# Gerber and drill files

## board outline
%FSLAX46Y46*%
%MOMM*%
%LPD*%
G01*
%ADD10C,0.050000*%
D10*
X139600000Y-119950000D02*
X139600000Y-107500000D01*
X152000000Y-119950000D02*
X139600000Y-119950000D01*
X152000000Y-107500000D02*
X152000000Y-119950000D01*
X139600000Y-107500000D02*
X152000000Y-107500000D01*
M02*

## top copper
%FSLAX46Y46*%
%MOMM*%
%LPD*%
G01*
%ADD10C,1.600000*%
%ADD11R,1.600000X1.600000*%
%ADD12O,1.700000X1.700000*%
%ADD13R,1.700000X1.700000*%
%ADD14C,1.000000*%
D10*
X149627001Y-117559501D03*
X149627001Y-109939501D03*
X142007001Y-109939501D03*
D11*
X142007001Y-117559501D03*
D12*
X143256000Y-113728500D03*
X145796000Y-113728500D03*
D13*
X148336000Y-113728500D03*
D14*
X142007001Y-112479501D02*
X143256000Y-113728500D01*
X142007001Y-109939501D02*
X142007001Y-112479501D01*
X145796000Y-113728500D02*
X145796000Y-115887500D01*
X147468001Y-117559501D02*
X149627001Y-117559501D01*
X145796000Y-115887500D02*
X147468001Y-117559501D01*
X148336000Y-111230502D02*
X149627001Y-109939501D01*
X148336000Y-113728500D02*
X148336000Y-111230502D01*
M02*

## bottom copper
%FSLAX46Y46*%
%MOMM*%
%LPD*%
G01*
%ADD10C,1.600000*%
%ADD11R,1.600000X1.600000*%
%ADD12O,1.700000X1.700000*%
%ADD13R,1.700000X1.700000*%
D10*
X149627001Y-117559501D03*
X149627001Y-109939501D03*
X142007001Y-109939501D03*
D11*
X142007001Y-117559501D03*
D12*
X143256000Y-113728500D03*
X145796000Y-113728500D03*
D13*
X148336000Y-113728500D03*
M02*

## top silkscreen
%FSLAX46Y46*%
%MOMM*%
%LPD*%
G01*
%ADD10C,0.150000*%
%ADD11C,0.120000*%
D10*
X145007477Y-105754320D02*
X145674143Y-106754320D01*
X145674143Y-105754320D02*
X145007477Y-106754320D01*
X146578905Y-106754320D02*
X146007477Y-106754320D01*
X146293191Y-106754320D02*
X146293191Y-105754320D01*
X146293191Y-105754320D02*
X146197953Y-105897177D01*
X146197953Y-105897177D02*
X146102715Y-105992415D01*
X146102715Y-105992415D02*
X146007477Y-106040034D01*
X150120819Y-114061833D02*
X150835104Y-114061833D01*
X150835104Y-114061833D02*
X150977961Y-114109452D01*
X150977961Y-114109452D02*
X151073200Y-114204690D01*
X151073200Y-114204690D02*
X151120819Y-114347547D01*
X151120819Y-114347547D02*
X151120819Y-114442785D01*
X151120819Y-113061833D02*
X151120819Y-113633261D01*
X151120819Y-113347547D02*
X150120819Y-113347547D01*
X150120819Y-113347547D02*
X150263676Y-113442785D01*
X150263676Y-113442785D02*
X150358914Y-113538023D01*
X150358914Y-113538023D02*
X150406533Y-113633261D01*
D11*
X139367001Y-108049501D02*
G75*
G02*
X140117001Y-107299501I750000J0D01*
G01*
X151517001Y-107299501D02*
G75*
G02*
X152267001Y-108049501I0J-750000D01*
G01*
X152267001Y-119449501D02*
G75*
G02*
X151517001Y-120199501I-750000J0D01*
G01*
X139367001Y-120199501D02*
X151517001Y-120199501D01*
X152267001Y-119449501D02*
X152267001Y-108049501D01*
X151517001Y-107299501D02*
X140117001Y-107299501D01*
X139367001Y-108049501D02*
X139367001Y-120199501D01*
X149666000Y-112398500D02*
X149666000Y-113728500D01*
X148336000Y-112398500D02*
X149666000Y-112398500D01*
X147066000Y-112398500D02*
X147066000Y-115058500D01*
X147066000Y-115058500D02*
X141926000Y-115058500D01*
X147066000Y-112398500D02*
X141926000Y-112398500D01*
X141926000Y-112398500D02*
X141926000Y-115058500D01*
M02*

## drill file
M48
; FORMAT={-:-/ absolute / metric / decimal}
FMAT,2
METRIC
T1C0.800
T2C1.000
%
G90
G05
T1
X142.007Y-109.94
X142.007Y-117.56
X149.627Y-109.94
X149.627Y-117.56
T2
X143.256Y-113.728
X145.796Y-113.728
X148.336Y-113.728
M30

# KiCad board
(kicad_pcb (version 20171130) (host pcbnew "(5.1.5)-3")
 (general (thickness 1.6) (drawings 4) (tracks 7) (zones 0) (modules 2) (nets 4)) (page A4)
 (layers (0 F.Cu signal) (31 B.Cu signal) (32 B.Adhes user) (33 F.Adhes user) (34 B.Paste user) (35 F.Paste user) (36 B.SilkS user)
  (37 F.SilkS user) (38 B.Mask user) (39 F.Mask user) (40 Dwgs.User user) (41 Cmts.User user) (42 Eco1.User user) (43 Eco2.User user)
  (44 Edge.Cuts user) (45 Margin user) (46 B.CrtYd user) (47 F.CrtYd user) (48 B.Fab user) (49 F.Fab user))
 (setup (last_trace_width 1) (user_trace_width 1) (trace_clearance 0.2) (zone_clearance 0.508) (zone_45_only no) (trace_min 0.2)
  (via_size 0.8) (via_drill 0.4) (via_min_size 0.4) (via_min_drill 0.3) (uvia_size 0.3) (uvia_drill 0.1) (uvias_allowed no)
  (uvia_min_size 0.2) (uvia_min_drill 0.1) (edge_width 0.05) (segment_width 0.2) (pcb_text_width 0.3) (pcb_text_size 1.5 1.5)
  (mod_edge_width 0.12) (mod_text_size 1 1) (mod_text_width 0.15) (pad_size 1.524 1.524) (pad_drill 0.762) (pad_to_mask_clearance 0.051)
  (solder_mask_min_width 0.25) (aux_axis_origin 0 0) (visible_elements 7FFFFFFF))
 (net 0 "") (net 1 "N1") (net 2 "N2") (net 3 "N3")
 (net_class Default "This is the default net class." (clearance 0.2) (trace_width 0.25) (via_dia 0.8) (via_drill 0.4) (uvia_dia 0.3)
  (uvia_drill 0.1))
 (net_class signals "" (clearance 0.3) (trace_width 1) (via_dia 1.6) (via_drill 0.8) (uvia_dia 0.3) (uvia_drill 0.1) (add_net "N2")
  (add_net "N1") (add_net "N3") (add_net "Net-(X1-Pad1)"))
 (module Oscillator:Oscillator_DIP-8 (layer F.Cu) (at 142.007001 117.559501)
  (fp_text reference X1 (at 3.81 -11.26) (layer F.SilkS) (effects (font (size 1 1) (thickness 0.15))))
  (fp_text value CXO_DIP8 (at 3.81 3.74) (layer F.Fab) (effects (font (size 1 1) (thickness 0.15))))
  (fp_arc (start -1.89 -9.51) (end -2.64 -9.51) (angle 90) (layer F.SilkS) (width 0.12))
  (fp_arc (start 9.51 -9.51) (end 9.51 -10.26) (angle 90) (layer F.SilkS) (width 0.12))
  (fp_arc (start 9.51 1.89) (end 10.26 1.89) (angle 90) (layer F.SilkS) (width 0.12))
  (fp_line (start -2.64 2.64) (end 9.51 2.64) (layer F.SilkS) (width 0.12))
  (fp_line (start 10.26 1.89) (end 10.26 -9.51) (layer F.SilkS) (width 0.12))
  (fp_line (start 9.51 -10.26) (end -1.89 -10.26) (layer F.SilkS) (width 0.12))
  (fp_line (start -2.64 -9.51) (end -2.64 2.64) (layer F.SilkS) (width 0.12))
  (pad 4 thru_hole circle (at 7.62 0) (size 1.6 1.6) (drill 0.8) (layers *.Cu *.Mask) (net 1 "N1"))
  (pad 5 thru_hole circle (at 7.62 -7.62) (size 1.6 1.6) (drill 0.8) (layers *.Cu *.Mask) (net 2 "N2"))
  (pad 8 thru_hole circle (at 0 -7.62) (size 1.6 1.6) (drill 0.8) (layers *.Cu *.Mask) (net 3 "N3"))
  (pad 1 thru_hole rect (at 0 0) (size 1.6 1.6) (drill 0.8) (layers *.Cu *.Mask)))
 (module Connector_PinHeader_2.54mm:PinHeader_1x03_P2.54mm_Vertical (layer F.Cu) (at 148.336 113.7285 270)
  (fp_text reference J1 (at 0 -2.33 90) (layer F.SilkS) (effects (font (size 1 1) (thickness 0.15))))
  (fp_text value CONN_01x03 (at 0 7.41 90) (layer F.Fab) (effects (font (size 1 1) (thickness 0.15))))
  (fp_line (start -1.33 -1.33) (end 0 -1.33) (layer F.SilkS) (width 0.12))
  (fp_line (start -1.33 0) (end -1.33 -1.33) (layer F.SilkS) (width 0.12))
  (fp_line (start -1.33 1.27) (end 1.33 1.27) (layer F.SilkS) (width 0.12))
  (fp_line (start 1.33 1.27) (end 1.33 6.41) (layer F.SilkS) (width 0.12))
  (fp_line (start -1.33 1.27) (end -1.33 6.41) (layer F.SilkS) (width 0.12))
  (fp_line (start -1.33 6.41) (end 1.33 6.41) (layer F.SilkS) (width 0.12))
  (pad 3 thru_hole oval (at 0 5.08 270) (size 1.7 1.7) (drill 1) (layers *.Cu *.Mask) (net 3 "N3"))
  (pad 2 thru_hole oval (at 0 2.54 270) (size 1.7 1.7) (drill 1) (layers *.Cu *.Mask) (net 1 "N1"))
  (pad 1 thru_hole rect (at 0 0 270) (size 1.7 1.7) (drill 1) (layers *.Cu *.Mask) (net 2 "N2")))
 (gr_line (start 139.6 119.95) (end 139.6 107.5) (layer Edge.Cuts) (width 0.05))
 (gr_line (start 152 119.95) (end 139.6 119.95) (layer Edge.Cuts) (width 0.05))
 (gr_line (start 152 107.5) (end 152 119.95) (layer Edge.Cuts) (width 0.05))
 (gr_line (start 139.6 107.5) (end 152 107.5) (layer Edge.Cuts) (width 0.05))
 (segment (start 142.007001 112.479501) (end 143.256 113.7285) (width 1) (layer F.Cu) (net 3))
 (segment (start 142.007001 109.939501) (end 142.007001 112.479501) (width 1) (layer F.Cu) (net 3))
 (segment (start 145.796 113.7285) (end 145.796 115.8875) (width 1) (layer F.Cu) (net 1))
 (segment (start 147.468001 117.559501) (end 149.627001 117.559501) (width 1) (layer F.Cu) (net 1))
 (segment (start 145.796 115.8875) (end 147.468001 117.559501) (width 1) (layer F.Cu) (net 1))
 (segment (start 148.336 111.230502) (end 149.627001 109.939501) (width 1) (layer F.Cu) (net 2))
 (segment (start 148.336 113.7285) (end 148.336 111.230502) (width 1) (layer F.Cu) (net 2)))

